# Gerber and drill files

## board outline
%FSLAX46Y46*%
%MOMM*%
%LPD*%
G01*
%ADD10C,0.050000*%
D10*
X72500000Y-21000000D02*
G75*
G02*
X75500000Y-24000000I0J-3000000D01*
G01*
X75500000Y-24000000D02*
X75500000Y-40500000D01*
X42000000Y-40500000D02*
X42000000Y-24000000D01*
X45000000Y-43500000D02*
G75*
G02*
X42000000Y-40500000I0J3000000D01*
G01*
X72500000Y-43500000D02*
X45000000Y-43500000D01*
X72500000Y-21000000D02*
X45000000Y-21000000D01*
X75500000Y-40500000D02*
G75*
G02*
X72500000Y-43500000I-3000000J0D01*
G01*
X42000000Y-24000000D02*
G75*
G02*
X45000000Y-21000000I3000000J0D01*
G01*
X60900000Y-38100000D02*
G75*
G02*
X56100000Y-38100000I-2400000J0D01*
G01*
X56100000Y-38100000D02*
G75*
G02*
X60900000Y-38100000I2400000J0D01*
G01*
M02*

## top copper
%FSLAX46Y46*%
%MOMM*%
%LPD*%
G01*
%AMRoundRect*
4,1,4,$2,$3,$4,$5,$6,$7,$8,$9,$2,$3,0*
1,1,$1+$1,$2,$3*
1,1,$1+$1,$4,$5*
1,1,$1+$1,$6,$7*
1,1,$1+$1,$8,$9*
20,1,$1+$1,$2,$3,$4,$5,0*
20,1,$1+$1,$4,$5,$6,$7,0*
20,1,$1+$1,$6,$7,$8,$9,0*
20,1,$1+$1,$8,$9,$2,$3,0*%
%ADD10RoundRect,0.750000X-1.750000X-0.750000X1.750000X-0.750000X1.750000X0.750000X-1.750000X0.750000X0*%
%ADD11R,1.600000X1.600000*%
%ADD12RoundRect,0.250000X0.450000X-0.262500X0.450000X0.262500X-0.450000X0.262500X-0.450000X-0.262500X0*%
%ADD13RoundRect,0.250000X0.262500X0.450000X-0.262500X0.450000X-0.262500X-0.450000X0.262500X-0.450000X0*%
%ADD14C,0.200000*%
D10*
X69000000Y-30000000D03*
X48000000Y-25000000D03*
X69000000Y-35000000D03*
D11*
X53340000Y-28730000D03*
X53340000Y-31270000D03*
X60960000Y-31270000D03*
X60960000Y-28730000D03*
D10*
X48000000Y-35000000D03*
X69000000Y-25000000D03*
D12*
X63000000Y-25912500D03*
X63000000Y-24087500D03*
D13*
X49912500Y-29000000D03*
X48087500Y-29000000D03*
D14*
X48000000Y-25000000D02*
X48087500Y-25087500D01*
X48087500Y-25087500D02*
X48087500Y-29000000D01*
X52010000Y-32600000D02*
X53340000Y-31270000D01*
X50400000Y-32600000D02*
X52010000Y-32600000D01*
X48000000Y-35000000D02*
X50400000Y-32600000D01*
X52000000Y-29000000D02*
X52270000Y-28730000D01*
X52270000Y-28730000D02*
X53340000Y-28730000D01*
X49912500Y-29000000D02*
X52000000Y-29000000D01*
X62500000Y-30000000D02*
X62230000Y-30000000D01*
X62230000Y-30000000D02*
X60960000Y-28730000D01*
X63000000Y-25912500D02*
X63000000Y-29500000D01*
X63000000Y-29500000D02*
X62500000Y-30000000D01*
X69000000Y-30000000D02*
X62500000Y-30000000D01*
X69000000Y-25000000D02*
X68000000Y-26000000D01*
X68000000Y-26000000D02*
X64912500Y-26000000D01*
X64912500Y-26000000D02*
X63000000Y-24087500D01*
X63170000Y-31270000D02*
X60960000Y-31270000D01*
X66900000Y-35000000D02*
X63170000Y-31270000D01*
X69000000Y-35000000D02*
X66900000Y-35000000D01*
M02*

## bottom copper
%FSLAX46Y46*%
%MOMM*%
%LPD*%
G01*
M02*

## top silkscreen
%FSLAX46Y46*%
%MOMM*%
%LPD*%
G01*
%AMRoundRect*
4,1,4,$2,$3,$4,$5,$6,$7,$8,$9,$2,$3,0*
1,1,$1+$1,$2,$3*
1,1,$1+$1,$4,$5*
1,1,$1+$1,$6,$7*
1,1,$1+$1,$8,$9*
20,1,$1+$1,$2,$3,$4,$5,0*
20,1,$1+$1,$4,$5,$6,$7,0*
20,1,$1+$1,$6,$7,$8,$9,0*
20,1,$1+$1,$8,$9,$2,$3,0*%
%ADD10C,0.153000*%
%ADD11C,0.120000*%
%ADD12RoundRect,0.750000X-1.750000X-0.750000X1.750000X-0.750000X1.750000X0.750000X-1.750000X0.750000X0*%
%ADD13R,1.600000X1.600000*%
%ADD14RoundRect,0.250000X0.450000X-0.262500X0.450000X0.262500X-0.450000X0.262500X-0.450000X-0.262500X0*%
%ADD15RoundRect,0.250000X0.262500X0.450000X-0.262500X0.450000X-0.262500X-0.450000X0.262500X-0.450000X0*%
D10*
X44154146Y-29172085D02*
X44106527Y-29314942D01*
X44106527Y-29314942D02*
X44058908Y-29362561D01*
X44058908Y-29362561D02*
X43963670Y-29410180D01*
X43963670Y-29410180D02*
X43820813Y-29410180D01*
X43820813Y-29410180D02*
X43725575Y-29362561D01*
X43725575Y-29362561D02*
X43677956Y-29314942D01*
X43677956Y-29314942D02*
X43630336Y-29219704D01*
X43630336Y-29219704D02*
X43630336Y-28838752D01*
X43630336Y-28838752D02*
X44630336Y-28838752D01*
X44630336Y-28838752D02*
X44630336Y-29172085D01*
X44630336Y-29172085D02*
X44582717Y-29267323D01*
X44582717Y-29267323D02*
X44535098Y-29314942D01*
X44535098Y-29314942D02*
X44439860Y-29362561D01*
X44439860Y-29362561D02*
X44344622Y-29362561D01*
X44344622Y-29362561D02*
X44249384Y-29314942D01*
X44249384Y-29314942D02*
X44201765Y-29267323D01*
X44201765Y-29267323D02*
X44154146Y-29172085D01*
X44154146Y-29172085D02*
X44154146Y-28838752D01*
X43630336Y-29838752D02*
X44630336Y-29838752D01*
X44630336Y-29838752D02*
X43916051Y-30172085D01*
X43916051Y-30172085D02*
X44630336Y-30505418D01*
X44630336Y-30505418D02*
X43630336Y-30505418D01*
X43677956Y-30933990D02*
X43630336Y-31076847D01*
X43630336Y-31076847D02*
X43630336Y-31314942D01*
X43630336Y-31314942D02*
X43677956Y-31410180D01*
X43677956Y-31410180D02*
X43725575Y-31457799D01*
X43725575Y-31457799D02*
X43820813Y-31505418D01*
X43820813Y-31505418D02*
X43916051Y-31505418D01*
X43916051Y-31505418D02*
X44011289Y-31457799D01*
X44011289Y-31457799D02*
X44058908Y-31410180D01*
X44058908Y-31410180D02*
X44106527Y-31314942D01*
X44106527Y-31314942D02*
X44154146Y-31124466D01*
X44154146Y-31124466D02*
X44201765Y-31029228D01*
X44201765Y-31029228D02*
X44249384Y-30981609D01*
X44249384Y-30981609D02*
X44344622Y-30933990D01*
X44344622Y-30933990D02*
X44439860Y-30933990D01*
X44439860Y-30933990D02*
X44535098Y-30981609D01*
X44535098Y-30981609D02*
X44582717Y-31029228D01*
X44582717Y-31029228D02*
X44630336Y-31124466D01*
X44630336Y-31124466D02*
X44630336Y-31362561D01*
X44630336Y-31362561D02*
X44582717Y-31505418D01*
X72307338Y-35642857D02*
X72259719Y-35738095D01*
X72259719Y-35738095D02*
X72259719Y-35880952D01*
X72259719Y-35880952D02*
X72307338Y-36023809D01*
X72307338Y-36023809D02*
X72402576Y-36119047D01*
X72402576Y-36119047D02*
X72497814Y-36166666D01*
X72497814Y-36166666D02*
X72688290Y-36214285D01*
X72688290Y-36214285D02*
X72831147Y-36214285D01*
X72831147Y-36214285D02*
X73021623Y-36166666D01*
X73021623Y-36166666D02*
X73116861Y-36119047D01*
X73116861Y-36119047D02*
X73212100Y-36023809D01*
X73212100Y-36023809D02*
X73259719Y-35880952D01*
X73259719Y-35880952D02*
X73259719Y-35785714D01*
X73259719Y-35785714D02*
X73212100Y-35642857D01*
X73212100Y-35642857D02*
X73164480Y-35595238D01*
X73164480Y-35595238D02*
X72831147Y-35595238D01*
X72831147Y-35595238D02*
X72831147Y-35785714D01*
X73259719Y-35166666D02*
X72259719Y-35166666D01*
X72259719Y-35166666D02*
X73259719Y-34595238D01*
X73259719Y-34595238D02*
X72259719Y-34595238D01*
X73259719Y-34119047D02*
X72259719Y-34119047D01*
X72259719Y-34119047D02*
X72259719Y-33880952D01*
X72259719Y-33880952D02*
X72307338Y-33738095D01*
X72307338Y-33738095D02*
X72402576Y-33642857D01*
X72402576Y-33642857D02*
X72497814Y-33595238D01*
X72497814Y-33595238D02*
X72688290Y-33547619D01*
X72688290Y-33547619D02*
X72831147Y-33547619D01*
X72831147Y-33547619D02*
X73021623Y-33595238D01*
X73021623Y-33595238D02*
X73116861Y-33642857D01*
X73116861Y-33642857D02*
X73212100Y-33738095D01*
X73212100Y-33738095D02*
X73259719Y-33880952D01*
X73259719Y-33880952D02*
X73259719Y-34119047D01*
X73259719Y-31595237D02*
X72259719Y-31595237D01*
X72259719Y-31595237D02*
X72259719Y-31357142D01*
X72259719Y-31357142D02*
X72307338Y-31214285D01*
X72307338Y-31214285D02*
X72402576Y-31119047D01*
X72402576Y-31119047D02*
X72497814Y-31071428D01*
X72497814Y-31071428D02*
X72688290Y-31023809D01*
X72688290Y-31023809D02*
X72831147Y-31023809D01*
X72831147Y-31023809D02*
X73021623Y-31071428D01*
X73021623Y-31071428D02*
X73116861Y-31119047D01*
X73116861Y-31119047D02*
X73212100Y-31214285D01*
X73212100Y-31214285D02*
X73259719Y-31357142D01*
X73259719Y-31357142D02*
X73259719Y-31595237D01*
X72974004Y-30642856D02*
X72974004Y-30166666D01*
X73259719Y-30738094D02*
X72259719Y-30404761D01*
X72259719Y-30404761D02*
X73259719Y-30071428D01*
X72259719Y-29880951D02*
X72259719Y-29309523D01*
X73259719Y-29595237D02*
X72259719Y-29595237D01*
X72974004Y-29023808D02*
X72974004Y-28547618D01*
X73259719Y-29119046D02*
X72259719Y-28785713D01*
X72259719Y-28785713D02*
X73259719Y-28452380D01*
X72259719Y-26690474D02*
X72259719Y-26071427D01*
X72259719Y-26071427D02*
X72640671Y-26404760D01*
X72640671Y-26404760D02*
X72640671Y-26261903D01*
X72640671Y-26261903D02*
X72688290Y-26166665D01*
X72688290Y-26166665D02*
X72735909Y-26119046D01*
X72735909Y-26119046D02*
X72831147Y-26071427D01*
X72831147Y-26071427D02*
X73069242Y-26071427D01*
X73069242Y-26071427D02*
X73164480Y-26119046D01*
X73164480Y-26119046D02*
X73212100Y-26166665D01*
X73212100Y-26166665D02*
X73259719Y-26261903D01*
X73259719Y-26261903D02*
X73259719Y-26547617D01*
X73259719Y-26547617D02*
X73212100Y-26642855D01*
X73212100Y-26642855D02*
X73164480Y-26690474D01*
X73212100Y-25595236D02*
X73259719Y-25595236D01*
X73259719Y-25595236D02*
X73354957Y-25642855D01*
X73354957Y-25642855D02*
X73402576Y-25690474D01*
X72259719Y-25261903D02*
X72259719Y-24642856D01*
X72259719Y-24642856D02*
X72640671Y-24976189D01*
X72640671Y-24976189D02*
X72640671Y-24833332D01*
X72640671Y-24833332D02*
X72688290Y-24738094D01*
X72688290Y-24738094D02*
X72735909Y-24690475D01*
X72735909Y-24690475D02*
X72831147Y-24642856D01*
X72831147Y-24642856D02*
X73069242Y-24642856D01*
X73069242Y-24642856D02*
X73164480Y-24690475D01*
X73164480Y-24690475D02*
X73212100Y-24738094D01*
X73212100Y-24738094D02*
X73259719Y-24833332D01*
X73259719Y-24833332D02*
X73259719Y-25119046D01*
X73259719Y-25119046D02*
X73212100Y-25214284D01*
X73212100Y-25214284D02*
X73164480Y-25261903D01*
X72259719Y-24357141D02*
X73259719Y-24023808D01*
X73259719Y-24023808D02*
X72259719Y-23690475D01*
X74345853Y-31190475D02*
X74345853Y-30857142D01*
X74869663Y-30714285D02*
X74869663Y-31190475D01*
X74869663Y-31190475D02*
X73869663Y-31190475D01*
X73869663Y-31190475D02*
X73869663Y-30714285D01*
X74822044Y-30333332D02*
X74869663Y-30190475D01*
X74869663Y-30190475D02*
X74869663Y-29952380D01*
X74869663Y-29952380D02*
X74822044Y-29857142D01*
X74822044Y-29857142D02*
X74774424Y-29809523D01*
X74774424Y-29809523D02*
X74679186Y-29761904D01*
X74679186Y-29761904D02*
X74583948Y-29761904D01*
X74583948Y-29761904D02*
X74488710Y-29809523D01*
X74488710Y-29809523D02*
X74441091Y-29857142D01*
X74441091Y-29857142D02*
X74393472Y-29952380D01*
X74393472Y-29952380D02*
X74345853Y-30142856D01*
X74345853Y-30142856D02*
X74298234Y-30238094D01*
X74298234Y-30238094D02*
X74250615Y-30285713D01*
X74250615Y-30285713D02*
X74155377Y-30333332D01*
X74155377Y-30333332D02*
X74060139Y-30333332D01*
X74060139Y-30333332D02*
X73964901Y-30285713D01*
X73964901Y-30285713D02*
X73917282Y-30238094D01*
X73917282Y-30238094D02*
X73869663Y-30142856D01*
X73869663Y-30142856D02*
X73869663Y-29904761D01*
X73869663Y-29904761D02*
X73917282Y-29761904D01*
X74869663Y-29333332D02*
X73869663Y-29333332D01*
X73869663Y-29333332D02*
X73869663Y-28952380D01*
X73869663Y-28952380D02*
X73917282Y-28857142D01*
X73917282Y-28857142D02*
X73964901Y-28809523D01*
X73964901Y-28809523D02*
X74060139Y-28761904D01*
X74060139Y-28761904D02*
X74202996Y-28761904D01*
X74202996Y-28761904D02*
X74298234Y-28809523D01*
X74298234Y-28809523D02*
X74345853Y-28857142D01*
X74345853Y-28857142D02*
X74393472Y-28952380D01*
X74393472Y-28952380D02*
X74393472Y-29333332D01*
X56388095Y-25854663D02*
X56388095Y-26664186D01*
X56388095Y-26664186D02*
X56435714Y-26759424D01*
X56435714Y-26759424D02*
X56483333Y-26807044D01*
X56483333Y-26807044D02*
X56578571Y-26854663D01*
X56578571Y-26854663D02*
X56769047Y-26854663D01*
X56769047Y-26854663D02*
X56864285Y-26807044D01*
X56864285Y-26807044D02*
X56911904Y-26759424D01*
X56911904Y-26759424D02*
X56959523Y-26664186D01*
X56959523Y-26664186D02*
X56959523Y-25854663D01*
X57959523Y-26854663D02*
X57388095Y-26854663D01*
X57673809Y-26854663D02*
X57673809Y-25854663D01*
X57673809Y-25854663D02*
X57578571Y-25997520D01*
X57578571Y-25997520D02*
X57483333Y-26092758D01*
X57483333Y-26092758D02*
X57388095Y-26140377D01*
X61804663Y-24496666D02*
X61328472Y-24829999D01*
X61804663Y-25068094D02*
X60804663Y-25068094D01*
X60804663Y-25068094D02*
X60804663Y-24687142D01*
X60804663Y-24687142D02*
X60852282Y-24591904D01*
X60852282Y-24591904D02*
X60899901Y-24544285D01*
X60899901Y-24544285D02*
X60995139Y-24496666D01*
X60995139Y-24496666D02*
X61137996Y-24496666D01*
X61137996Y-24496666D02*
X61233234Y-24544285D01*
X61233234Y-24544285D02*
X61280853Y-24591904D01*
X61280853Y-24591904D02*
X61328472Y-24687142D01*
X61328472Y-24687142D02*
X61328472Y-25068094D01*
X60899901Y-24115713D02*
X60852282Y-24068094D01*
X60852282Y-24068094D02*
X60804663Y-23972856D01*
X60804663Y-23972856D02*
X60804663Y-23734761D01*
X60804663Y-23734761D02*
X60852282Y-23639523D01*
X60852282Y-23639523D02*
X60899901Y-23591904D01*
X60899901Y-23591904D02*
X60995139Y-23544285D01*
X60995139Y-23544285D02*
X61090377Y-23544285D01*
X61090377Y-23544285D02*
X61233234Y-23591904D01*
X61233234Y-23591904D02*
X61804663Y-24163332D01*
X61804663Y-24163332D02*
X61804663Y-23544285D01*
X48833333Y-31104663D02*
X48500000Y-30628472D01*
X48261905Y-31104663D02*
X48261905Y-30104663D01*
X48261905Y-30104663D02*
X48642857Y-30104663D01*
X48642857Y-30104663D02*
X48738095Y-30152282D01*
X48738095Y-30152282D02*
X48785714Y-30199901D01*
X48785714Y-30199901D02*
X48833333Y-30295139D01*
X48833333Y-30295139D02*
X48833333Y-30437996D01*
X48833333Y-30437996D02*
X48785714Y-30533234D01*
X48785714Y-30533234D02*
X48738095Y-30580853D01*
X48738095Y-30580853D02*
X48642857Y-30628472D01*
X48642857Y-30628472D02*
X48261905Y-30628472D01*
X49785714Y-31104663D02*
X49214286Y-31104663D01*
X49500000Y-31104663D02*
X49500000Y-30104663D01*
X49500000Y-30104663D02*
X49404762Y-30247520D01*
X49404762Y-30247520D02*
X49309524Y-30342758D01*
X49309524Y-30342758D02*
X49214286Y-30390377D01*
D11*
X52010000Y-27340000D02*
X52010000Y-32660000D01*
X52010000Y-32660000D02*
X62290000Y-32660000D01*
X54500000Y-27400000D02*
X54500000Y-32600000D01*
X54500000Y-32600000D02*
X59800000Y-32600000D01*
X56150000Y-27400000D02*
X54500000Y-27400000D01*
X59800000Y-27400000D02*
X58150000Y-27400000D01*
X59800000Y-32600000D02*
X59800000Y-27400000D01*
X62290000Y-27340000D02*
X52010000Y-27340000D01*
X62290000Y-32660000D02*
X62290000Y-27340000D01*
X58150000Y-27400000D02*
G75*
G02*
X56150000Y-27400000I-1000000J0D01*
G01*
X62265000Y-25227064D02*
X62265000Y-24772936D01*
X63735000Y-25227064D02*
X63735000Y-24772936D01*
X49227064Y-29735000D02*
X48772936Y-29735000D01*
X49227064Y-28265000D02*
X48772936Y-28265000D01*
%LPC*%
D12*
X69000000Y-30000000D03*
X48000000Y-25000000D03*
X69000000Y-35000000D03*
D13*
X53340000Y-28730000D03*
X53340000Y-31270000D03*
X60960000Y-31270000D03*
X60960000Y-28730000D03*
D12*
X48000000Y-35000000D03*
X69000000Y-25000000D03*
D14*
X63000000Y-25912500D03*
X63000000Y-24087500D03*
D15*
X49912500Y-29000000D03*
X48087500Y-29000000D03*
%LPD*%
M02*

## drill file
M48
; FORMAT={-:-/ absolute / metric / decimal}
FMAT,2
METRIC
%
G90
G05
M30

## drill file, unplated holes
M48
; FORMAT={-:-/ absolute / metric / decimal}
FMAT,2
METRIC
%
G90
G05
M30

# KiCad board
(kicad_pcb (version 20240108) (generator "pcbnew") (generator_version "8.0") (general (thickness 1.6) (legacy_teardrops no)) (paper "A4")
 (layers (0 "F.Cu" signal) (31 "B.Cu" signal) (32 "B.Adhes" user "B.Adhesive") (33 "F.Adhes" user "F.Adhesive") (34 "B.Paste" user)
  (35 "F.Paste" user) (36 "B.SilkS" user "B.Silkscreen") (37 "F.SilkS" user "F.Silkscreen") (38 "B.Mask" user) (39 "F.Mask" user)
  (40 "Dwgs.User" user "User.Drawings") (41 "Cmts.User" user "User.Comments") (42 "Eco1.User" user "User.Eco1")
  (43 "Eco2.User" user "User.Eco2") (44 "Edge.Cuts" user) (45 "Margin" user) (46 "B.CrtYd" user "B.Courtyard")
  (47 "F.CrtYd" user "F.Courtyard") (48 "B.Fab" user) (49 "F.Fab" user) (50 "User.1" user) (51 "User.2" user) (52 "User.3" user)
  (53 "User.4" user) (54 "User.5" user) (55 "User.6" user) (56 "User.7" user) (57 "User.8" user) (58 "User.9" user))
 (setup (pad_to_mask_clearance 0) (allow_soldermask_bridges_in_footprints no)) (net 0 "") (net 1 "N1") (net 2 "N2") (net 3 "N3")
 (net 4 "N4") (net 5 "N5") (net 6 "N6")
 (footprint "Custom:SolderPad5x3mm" (layer "F.Cu") (at 69 25)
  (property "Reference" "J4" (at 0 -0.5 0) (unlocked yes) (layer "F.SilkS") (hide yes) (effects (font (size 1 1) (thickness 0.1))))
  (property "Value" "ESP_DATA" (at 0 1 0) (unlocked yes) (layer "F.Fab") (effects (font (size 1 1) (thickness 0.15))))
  (pad "1" smd roundrect (at 0 5) (size 5 3) (layers "F.Cu" "F.Paste" "F.Mask") (roundrect_rratio 0.25) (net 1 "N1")
   (thermal_bridge_angle 45)))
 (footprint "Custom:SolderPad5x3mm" (layer "F.Cu") (at 48 20)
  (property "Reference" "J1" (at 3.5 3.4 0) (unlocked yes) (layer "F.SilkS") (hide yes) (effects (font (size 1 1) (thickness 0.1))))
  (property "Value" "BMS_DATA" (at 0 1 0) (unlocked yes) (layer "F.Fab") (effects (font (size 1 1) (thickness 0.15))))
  (pad "1" smd roundrect (at 0 5) (size 5 3) (layers "F.Cu" "F.Paste" "F.Mask") (roundrect_rratio 0.25) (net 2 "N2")
   (thermal_bridge_angle 45)))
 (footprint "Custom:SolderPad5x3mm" (layer "F.Cu") (at 69 30)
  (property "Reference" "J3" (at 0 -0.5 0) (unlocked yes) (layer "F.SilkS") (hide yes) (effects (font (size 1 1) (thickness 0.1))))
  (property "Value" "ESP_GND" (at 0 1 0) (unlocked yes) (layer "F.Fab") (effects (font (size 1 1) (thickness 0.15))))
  (pad "1" smd roundrect (at 0 5) (size 5 3) (layers "F.Cu" "F.Paste" "F.Mask") (roundrect_rratio 0.25) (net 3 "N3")
   (thermal_bridge_angle 45)))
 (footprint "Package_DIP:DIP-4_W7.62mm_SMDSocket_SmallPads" (layer "F.Cu") (at 57.15 30)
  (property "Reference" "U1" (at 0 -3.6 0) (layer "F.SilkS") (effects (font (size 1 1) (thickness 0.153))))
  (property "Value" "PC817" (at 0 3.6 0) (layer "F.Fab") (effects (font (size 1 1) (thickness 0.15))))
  (fp_line (start -5.14 -2.66) (end -5.14 2.66) (stroke (width 0.12) (type solid)) (layer "F.SilkS"))
  (fp_line (start -5.14 2.66) (end 5.14 2.66) (stroke (width 0.12) (type solid)) (layer "F.SilkS"))
  (fp_line (start -2.65 -2.6) (end -2.65 2.6) (stroke (width 0.12) (type solid)) (layer "F.SilkS"))
  (fp_line (start -2.65 2.6) (end 2.65 2.6) (stroke (width 0.12) (type solid)) (layer "F.SilkS"))
  (fp_line (start -1 -2.6) (end -2.65 -2.6) (stroke (width 0.12) (type solid)) (layer "F.SilkS"))
  (fp_line (start 2.65 -2.6) (end 1 -2.6) (stroke (width 0.12) (type solid)) (layer "F.SilkS"))
  (fp_line (start 2.65 2.6) (end 2.65 -2.6) (stroke (width 0.12) (type solid)) (layer "F.SilkS"))
  (fp_line (start 5.14 -2.66) (end -5.14 -2.66) (stroke (width 0.12) (type solid)) (layer "F.SilkS"))
  (fp_line (start 5.14 2.66) (end 5.14 -2.66) (stroke (width 0.12) (type solid)) (layer "F.SilkS"))
  (fp_arc (start 1 -2.6) (mid 0 -1.6) (end -1 -2.6) (stroke (width 0.12) (type solid)) (layer "F.SilkS"))
  (pad "1" smd rect (at -3.81 -1.27) (size 1.6 1.6) (layers "F.Cu" "F.Paste" "F.Mask") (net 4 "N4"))
  (pad "2" smd rect (at -3.81 1.27) (size 1.6 1.6) (layers "F.Cu" "F.Paste" "F.Mask") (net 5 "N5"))
  (pad "3" smd rect (at 3.81 1.27) (size 1.6 1.6) (layers "F.Cu" "F.Paste" "F.Mask") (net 3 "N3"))
  (pad "4" smd rect (at 3.81 -1.27) (size 1.6 1.6) (layers "F.Cu" "F.Paste" "F.Mask") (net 1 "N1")))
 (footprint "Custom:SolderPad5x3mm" (layer "F.Cu") (at 48 30)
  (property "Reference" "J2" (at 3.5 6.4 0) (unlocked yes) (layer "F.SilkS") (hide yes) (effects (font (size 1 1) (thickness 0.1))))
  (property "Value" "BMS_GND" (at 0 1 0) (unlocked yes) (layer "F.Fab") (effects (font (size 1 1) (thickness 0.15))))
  (pad "1" smd roundrect (at 0 5) (size 5 3) (layers "F.Cu" "F.Paste" "F.Mask") (roundrect_rratio 0.25) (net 5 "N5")
   (thermal_bridge_angle 45)))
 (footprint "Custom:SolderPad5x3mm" (layer "F.Cu") (at 69 20)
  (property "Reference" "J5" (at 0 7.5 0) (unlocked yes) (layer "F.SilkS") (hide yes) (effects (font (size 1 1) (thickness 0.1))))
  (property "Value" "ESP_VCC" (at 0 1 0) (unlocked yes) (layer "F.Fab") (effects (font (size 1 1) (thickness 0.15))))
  (pad "1" smd roundrect (at 0 5) (size 5 3) (layers "F.Cu" "F.Paste" "F.Mask") (roundrect_rratio 0.25) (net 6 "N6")
   (thermal_bridge_angle 45)))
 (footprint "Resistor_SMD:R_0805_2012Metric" (layer "F.Cu") (at 63 25 90)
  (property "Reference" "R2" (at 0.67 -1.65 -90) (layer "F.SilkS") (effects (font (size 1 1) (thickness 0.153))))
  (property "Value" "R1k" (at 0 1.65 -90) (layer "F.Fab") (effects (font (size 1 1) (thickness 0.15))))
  (fp_line (start -0.227064 -0.735) (end 0.227064 -0.735) (stroke (width 0.12) (type solid)) (layer "F.SilkS"))
  (fp_line (start -0.227064 0.735) (end 0.227064 0.735) (stroke (width 0.12) (type solid)) (layer "F.SilkS"))
  (pad "1" smd roundrect (at -0.9125 0 90) (size 1.025 1.4) (layers "F.Cu" "F.Paste" "F.Mask") (roundrect_rratio 0.243902) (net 1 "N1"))
  (pad "2" smd roundrect (at 0.9125 0 90) (size 1.025 1.4) (layers "F.Cu" "F.Paste" "F.Mask") (roundrect_rratio 0.243902) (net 6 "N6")))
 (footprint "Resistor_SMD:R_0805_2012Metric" (layer "F.Cu") (at 49 29 180)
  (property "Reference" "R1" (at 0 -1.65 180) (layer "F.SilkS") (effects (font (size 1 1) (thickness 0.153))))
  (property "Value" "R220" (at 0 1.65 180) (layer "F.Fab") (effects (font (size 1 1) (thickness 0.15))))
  (fp_line (start -0.227064 0.735) (end 0.227064 0.735) (stroke (width 0.12) (type solid)) (layer "F.SilkS"))
  (fp_line (start -0.227064 -0.735) (end 0.227064 -0.735) (stroke (width 0.12) (type solid)) (layer "F.SilkS"))
  (pad "1" smd roundrect (at -0.9125 0 180) (size 1.025 1.4) (layers "F.Cu" "F.Paste" "F.Mask") (roundrect_rratio 0.243902) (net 4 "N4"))
  (pad "2" smd roundrect (at 0.9125 0 180) (size 1.025 1.4) (layers "F.Cu" "F.Paste" "F.Mask") (roundrect_rratio 0.243902) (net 2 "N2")))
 (gr_arc (start 72.5 21) (mid 74.62132 21.87868) (end 75.5 24) (stroke (width 0.05) (type default)) (layer "Edge.Cuts"))
 (gr_line (start 75.5 24) (end 75.5 40.5) (stroke (width 0.05) (type default)) (layer "Edge.Cuts"))
 (gr_line (start 42 40.5) (end 42 24) (stroke (width 0.05) (type default)) (layer "Edge.Cuts"))
 (gr_arc (start 45 43.5) (mid 42.87868 42.62132) (end 42 40.5) (stroke (width 0.05) (type default)) (layer "Edge.Cuts"))
 (gr_line (start 72.5 43.5) (end 45 43.5) (stroke (width 0.05) (type default)) (layer "Edge.Cuts"))
 (gr_line (start 72.5 21) (end 45 21) (stroke (width 0.05) (type default)) (layer "Edge.Cuts"))
 (gr_arc (start 75.5 40.5) (mid 74.62132 42.62132) (end 72.5 43.5) (stroke (width 0.05) (type default)) (layer "Edge.Cuts"))
 (gr_arc (start 42 24) (mid 42.87868 21.87868) (end 45 21) (stroke (width 0.05) (type default)) (layer "Edge.Cuts"))
 (gr_circle (center 58.5 38.1) (end 60.9 38.1) (stroke (width 0.05) (type default)) (fill none) (layer "Edge.Cuts"))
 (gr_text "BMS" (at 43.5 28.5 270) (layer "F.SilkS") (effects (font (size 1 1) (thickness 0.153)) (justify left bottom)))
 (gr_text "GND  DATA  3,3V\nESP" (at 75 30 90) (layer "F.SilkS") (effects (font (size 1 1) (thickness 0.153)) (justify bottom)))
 (segment (start 48 25) (end 48.0875 25.0875) (width 0.2) (layer "F.Cu") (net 2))
 (segment (start 48.0875 25.0875) (end 48.0875 29) (width 0.2) (layer "F.Cu") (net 2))
 (segment (start 52.01 32.6) (end 53.34 31.27) (width 0.2) (layer "F.Cu") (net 5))
 (segment (start 50.4 32.6) (end 52.01 32.6) (width 0.2) (layer "F.Cu") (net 5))
 (segment (start 48 35) (end 50.4 32.6) (width 0.2) (layer "F.Cu") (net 5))
 (segment (start 52 29) (end 52.27 28.73) (width 0.2) (layer "F.Cu") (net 4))
 (segment (start 52.27 28.73) (end 53.34 28.73) (width 0.2) (layer "F.Cu") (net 4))
 (segment (start 49.9125 29) (end 52 29) (width 0.2) (layer "F.Cu") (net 4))
 (segment (start 62.5 30) (end 62.23 30) (width 0.2) (layer "F.Cu") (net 1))
 (segment (start 62.23 30) (end 60.96 28.73) (width 0.2) (layer "F.Cu") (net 1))
 (segment (start 63 25.9125) (end 63 29.5) (width 0.2) (layer "F.Cu") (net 1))
 (segment (start 63 29.5) (end 62.5 30) (width 0.2) (layer "F.Cu") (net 1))
 (segment (start 69 30) (end 62.5 30) (width 0.2) (layer "F.Cu") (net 1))
 (segment (start 69 25) (end 68 26) (width 0.2) (layer "F.Cu") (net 6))
 (segment (start 68 26) (end 64.9125 26) (width 0.2) (layer "F.Cu") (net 6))
 (segment (start 64.9125 26) (end 63 24.0875) (width 0.2) (layer "F.Cu") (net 6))
 (segment (start 63.17 31.27) (end 60.96 31.27) (width 0.2) (layer "F.Cu") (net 3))
 (segment (start 66.9 35) (end 63.17 31.27) (width 0.2) (layer "F.Cu") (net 3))
 (segment (start 69 35) (end 66.9 35) (width 0.2) (layer "F.Cu") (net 3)))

